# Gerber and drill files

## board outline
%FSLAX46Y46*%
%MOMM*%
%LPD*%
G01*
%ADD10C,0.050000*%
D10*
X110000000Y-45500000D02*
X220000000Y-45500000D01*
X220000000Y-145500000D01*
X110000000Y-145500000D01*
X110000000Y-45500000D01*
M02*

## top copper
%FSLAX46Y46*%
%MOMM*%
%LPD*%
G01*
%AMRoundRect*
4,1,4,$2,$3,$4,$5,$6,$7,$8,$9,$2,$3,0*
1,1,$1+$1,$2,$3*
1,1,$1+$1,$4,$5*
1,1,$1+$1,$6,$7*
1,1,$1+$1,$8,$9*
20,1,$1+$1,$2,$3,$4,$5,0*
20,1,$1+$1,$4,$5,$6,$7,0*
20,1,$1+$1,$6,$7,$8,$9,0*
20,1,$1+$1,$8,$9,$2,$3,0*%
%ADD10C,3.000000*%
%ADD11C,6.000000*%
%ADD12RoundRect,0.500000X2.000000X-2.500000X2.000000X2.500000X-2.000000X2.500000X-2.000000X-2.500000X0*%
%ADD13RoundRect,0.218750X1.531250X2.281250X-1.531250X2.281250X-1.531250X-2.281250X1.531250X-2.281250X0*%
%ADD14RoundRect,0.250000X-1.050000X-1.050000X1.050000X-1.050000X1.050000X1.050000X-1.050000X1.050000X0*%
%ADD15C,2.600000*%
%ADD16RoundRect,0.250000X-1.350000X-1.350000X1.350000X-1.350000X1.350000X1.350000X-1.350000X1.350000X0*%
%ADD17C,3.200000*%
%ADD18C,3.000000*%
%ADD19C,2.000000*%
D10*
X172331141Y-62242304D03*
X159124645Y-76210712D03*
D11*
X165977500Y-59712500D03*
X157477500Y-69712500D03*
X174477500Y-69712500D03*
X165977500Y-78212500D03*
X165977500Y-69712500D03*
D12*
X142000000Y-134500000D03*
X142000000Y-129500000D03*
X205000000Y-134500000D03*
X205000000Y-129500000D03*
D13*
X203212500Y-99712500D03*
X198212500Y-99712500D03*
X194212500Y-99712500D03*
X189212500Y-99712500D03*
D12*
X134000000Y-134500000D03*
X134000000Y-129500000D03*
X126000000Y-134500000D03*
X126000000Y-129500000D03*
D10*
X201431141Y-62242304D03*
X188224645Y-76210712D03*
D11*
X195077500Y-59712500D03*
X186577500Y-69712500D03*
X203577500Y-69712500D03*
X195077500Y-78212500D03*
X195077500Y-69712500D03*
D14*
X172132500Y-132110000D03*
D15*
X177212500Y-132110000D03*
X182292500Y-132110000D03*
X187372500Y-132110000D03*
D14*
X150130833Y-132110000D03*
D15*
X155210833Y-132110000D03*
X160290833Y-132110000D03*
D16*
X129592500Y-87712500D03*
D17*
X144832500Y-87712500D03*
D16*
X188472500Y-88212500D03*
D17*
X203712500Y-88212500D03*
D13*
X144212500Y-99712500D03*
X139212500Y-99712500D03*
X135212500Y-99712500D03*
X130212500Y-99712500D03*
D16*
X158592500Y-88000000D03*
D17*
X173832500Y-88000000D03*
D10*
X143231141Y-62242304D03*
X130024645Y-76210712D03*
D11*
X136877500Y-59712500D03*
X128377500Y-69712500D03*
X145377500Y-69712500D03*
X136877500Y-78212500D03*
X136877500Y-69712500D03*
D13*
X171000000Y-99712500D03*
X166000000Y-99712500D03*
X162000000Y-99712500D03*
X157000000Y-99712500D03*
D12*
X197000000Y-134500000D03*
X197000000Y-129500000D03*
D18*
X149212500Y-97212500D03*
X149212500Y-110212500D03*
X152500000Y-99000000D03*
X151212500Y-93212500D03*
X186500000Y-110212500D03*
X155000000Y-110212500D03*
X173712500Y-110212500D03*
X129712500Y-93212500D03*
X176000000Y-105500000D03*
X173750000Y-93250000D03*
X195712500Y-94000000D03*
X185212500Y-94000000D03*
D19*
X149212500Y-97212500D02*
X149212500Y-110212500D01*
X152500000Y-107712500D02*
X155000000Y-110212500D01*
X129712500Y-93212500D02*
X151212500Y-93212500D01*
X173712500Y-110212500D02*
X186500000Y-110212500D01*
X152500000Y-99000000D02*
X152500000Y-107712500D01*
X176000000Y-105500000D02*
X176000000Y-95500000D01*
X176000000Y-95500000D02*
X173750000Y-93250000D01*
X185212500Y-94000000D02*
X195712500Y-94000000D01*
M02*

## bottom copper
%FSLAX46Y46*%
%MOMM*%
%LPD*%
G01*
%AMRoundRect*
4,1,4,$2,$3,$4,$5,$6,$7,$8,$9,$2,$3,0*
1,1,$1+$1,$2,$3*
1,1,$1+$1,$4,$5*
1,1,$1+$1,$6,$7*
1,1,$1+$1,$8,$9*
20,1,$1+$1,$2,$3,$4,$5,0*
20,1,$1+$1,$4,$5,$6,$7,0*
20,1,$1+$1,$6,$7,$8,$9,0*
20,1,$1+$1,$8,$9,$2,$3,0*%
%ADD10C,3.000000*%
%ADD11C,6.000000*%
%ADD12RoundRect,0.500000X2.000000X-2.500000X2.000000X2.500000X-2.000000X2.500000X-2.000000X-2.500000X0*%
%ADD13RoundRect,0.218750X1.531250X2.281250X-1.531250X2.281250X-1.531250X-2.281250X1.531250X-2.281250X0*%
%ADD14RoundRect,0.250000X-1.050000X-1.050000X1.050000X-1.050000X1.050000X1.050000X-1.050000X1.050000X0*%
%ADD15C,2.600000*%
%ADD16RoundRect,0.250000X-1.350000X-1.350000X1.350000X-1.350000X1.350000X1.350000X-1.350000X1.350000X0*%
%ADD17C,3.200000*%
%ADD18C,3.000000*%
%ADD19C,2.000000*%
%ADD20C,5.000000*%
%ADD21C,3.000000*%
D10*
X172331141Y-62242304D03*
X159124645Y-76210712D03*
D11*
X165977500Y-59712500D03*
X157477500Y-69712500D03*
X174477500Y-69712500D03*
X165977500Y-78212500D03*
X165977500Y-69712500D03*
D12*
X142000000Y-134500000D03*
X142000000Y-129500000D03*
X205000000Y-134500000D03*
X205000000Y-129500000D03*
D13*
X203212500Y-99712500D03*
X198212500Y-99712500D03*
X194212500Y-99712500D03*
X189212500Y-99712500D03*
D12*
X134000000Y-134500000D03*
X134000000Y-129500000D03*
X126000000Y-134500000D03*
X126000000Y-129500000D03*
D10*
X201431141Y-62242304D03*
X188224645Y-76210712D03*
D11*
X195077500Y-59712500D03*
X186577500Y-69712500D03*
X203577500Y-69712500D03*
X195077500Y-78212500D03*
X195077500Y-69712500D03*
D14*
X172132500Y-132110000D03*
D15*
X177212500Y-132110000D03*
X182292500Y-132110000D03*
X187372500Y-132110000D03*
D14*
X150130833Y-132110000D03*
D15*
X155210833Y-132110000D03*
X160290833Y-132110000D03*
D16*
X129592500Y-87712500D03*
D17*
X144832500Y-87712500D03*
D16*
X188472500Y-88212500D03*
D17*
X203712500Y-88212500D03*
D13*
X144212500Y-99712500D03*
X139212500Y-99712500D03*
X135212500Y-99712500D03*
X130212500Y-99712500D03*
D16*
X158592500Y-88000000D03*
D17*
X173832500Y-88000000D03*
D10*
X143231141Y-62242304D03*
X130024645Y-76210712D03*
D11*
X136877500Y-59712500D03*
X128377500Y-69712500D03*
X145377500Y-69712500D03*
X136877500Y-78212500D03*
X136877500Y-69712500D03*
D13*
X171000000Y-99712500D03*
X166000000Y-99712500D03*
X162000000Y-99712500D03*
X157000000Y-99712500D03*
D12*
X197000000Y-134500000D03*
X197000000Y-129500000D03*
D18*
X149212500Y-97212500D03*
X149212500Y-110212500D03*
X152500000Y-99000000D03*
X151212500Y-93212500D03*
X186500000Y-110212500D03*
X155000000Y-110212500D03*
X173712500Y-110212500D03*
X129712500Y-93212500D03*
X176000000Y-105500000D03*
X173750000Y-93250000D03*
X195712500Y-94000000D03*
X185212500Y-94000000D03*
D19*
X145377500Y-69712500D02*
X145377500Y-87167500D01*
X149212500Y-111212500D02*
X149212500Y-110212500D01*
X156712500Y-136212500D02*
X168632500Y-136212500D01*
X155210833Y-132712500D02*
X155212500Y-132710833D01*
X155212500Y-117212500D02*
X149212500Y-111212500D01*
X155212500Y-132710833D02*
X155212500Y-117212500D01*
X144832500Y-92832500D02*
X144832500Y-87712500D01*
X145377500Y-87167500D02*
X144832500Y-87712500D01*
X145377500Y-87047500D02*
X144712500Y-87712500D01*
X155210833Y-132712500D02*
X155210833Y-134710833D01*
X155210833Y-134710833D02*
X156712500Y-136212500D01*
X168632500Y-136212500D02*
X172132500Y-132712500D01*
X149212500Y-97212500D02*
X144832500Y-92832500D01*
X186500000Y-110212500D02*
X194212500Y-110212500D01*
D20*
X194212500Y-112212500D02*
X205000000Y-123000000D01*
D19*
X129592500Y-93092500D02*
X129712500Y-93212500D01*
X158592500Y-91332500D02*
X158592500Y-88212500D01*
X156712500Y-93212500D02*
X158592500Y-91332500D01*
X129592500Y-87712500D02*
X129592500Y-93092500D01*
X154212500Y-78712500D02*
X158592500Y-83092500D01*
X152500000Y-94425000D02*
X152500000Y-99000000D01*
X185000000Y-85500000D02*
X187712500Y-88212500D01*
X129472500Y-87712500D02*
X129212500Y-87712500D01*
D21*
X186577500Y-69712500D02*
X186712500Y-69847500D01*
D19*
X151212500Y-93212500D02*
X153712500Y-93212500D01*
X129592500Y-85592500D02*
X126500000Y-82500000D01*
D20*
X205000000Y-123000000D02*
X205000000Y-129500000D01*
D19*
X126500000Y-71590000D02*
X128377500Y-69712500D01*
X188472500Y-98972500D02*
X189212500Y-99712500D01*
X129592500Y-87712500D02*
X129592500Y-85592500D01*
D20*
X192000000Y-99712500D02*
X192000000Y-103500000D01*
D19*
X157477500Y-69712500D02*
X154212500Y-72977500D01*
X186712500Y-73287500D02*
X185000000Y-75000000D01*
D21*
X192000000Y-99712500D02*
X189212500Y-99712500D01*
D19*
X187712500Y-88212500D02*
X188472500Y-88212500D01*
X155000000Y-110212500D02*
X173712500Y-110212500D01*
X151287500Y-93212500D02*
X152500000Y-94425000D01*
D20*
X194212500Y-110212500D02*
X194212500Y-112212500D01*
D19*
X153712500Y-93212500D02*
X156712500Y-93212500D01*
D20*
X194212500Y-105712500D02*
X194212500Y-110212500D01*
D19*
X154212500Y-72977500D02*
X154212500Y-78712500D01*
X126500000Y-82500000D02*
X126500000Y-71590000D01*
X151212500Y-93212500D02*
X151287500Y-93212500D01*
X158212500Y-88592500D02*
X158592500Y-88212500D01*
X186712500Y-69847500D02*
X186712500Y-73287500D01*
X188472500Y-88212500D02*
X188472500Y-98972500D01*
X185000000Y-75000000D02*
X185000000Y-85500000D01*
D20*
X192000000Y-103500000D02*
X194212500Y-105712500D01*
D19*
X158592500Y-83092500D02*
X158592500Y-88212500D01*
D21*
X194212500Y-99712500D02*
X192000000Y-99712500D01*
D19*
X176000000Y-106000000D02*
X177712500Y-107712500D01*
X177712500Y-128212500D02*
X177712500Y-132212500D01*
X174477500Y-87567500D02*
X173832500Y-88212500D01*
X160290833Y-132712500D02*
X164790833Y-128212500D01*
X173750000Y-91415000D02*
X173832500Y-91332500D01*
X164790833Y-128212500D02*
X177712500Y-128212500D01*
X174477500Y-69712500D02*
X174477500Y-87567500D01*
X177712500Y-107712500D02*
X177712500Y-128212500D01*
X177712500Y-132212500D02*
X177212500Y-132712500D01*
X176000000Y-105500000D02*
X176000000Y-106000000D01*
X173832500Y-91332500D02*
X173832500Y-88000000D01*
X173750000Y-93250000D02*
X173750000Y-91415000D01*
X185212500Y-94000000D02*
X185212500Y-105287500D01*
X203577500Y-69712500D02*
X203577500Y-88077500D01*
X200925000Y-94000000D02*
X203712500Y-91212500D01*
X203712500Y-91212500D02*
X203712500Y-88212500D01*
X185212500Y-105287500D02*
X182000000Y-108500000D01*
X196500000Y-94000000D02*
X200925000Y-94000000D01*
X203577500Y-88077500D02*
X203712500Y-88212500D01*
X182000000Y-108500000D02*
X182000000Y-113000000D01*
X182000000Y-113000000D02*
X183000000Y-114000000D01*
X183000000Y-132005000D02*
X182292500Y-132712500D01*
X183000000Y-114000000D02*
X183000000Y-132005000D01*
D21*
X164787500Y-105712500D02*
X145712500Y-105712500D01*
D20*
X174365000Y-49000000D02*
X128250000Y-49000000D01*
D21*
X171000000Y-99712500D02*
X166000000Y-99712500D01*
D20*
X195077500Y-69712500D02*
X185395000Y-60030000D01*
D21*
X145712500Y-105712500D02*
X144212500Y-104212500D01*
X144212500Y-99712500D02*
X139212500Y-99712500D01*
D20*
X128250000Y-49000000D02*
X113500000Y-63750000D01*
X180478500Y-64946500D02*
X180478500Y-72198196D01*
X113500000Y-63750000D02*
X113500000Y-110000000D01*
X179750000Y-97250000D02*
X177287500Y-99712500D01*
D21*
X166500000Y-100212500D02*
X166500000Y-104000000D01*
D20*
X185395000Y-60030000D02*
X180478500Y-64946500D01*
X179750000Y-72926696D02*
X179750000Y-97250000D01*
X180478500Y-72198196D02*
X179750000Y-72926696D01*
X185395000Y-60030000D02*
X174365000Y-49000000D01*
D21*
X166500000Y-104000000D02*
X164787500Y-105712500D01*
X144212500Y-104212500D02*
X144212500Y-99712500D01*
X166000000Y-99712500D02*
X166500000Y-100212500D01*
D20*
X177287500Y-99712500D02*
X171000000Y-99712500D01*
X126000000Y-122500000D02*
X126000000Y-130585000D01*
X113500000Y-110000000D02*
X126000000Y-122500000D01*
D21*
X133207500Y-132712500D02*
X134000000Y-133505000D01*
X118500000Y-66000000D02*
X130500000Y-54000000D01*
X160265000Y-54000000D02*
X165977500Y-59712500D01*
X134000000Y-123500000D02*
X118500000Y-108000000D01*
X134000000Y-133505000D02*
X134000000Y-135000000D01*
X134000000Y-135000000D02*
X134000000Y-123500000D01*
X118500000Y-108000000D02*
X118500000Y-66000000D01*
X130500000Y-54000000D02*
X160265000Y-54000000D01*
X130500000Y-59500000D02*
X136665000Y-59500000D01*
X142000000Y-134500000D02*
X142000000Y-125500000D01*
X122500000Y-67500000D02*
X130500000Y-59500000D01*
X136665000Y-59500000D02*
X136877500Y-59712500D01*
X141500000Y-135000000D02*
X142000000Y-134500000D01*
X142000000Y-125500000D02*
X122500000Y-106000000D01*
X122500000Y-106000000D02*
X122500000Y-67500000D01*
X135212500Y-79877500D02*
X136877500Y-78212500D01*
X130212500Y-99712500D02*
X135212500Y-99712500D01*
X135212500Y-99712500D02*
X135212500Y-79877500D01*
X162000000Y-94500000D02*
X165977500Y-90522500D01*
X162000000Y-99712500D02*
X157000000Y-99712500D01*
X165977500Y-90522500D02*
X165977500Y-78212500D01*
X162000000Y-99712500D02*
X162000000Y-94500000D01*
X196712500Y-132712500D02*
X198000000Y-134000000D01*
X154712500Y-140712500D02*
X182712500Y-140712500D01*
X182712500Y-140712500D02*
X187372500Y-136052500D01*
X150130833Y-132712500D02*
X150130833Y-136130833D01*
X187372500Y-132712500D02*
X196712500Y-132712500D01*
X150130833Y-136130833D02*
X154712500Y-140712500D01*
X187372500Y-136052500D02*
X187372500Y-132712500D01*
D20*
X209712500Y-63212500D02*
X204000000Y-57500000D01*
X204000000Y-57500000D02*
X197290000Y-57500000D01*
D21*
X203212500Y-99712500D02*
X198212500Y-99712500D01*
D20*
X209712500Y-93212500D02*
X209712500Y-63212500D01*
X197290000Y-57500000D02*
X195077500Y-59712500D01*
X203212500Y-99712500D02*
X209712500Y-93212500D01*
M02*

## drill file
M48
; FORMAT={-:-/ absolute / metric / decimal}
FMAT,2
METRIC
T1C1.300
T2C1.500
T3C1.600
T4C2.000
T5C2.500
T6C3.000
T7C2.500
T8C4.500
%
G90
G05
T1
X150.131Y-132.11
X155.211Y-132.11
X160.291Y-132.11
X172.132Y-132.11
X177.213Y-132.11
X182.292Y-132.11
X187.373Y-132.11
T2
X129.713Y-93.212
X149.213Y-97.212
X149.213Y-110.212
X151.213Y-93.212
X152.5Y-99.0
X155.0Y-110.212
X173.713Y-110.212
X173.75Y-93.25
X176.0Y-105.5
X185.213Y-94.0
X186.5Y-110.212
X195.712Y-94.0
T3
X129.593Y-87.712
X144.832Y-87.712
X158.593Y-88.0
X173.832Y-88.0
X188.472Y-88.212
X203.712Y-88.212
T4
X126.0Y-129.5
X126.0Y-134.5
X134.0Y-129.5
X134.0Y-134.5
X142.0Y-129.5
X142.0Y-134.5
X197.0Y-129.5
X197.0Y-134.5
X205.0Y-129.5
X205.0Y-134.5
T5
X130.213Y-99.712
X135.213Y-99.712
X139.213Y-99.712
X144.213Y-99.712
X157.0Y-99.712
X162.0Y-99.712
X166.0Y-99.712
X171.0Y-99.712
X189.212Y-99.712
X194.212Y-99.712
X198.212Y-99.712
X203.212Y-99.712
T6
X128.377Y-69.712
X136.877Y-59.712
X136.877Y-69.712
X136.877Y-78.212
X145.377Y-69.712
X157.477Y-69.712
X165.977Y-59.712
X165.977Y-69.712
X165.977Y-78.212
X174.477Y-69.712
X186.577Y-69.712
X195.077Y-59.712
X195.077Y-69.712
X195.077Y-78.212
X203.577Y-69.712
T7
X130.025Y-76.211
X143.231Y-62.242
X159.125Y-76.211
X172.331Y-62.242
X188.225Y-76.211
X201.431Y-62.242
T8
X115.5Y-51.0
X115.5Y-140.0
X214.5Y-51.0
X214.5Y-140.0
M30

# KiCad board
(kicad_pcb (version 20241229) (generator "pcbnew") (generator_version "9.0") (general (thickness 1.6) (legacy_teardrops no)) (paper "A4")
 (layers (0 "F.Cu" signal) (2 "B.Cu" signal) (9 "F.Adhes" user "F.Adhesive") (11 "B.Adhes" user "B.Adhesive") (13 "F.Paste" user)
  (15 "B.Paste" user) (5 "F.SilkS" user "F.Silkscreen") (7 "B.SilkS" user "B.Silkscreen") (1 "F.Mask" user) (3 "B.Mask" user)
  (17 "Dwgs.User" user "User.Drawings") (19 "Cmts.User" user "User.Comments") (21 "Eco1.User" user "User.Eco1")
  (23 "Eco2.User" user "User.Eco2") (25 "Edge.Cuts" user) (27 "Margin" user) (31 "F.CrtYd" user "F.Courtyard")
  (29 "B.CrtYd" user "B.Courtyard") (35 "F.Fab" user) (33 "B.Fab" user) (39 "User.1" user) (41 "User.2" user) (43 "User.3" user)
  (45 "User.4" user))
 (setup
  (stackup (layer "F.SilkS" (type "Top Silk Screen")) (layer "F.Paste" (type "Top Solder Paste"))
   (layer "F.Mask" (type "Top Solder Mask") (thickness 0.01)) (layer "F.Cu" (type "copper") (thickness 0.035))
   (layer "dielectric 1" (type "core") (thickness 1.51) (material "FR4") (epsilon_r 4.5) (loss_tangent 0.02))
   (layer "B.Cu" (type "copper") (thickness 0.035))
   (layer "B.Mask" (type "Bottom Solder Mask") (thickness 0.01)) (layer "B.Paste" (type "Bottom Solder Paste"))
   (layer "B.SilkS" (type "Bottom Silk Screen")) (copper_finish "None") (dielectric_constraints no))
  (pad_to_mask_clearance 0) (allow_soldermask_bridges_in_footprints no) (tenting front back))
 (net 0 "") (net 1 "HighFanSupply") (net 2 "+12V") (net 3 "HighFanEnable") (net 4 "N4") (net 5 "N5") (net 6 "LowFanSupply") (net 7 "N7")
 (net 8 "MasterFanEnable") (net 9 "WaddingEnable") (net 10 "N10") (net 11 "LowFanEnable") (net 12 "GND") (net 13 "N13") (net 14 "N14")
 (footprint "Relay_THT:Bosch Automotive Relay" (layer "F.Cu") (at 165.9775 69.4625 180)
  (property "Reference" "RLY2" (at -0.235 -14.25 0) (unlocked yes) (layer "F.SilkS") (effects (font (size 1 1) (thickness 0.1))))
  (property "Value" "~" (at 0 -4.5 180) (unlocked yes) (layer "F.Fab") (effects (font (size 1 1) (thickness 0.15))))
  (pad "" np_thru_hole circle (at -6.353641 7.220196 180) (size 3 3) (drill 2.5) (layers "*.Cu" "*.Mask"))
  (pad "" np_thru_hole circle (at 6.852855 -6.748212 180) (size 3 3) (drill 2.5) (layers "*.Cu" "*.Mask"))
  (pad "30" thru_hole circle (at 0 9.75 180) (size 6 6) (drill 3) (layers "*.Cu" "*.Mask") (remove_unused_layers no) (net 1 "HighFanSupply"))
  (pad "85" thru_hole circle (at 8.5 -0.25 180) (size 6 6) (drill 3) (layers "*.Cu" "*.Mask") (remove_unused_layers no) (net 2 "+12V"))
  (pad "86" thru_hole circle (at -8.5 -0.25 180) (size 6 6) (drill 3) (layers "*.Cu" "*.Mask") (remove_unused_layers no)
   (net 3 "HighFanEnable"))
  (pad "87" thru_hole circle (at 0 -8.75 180) (size 6 6) (drill 3) (layers "*.Cu" "*.Mask") (remove_unused_layers no) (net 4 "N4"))
  (pad "87a" thru_hole circle (at 0 -0.25 180) (size 6 6) (drill 3) (layers "*.Cu" "*.Mask") (remove_unused_layers no) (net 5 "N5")))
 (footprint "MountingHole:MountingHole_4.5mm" (layer "F.Cu") (at 115.5 51)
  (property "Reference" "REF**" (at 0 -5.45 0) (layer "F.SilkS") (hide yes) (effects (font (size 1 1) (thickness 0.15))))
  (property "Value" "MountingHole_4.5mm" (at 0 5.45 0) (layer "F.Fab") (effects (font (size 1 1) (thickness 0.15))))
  (pad "" np_thru_hole circle (at 0 0) (size 4.5 4.5) (drill 4.5) (layers "*.Cu" "*.Mask")))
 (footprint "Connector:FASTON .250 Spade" (layer "F.Cu") (at 142 132 90)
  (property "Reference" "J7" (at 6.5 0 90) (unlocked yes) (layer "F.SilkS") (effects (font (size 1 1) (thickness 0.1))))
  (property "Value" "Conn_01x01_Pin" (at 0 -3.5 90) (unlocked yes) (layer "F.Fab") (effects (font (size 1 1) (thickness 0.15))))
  (pad "1" thru_hole roundrect (at -2.5 0 90) (size 6 5) (drill 2) (layers "*.Cu" "*.Mask") (remove_unused_layers no) (roundrect_rratio 0.1)
   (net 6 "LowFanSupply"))
  (pad "1" thru_hole roundrect (at 2.5 0 90) (size 6 5) (drill 2) (layers "*.Cu" "*.Mask") (remove_unused_layers no) (roundrect_rratio 0.1)
   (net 6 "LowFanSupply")))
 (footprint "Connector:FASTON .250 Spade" (layer "F.Cu") (at 205 132 90)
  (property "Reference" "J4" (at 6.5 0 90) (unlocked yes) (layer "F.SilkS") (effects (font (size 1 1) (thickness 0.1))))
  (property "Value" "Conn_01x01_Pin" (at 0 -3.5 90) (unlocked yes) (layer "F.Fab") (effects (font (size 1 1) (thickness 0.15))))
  (pad "1" thru_hole roundrect (at -2.5 0 90) (size 6 5) (drill 2) (layers "*.Cu" "*.Mask") (remove_unused_layers no) (roundrect_rratio 0.1)
   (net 2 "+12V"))
  (pad "1" thru_hole roundrect (at 2.5 0 90) (size 6 5) (drill 2) (layers "*.Cu" "*.Mask") (remove_unused_layers no) (roundrect_rratio 0.1)
   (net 2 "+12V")))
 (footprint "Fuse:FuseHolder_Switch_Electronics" (layer "F.Cu") (at 196.2125 99.7125 180)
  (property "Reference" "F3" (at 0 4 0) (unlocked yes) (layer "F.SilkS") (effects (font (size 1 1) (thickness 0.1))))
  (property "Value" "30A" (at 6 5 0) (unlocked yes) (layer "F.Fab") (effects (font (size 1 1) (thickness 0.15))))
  (pad "1" thru_hole roundrect (at -7 0 180) (size 3.5 5) (drill 2.5) (layers "*.Cu" "*.Mask") (remove_unused_layers no)
   (roundrect_rratio 0.0625) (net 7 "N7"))
  (pad "1" thru_hole roundrect (at -2 0 180) (size 3.5 5) (drill 2.5) (layers "*.Cu" "*.Mask") (remove_unused_layers no)
   (roundrect_rratio 0.0625) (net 7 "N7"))
  (pad "2" thru_hole roundrect (at 2 0 180) (size 3.5 5) (drill 2.5) (layers "*.Cu" "*.Mask") (remove_unused_layers no)
   (roundrect_rratio 0.0625) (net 2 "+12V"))
  (pad "2" thru_hole roundrect (at 7 0 180) (size 3.5 5) (drill 2.5) (layers "*.Cu" "*.Mask") (remove_unused_layers no)
   (roundrect_rratio 0.0625) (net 2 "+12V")))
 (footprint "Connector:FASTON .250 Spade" (layer "F.Cu") (at 134 132 90)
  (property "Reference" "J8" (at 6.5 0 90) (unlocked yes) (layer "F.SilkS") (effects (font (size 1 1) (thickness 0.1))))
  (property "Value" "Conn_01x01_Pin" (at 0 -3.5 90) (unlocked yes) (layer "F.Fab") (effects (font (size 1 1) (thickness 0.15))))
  (pad "1" thru_hole roundrect (at -2.5 0 90) (size 6 5) (drill 2) (layers "*.Cu" "*.Mask") (remove_unused_layers no) (roundrect_rratio 0.1)
   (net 1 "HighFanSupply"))
  (pad "1" thru_hole roundrect (at 2.5 0 90) (size 6 5) (drill 2) (layers "*.Cu" "*.Mask") (remove_unused_layers no) (roundrect_rratio 0.1)
   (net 1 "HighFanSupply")))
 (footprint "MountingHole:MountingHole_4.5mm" (layer "F.Cu") (at 214.5 140)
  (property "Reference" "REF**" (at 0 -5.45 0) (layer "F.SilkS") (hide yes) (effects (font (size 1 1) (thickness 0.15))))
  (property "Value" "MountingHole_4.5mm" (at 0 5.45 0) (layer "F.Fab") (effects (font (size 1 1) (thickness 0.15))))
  (pad "" np_thru_hole circle (at 0 0) (size 4.5 4.5) (drill 4.5) (layers "*.Cu" "*.Mask")))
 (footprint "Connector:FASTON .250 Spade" (layer "F.Cu") (at 126 132 90)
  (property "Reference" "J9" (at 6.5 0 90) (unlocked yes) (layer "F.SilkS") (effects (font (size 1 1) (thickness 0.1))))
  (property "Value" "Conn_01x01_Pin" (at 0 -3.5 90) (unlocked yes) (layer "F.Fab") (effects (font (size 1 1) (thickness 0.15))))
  (pad "1" thru_hole roundrect (at -2.5 0 90) (size 6 5) (drill 2) (layers "*.Cu" "*.Mask") (remove_unused_layers no) (roundrect_rratio 0.1)
   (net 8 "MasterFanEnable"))
  (pad "1" thru_hole roundrect (at 2.5 0 90) (size 6 5) (drill 2) (layers "*.Cu" "*.Mask") (remove_unused_layers no) (roundrect_rratio 0.1)
   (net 8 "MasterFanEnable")))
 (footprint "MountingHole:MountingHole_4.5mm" (layer "F.Cu") (at 115.5 140)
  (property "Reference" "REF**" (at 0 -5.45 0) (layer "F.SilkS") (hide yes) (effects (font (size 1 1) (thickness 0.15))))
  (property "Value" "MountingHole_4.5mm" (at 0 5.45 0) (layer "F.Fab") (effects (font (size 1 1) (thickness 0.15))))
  (pad "" np_thru_hole circle (at 0 0) (size 4.5 4.5) (drill 4.5) (layers "*.Cu" "*.Mask")))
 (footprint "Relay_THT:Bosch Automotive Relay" (layer "F.Cu") (at 195.0775 69.4625 180)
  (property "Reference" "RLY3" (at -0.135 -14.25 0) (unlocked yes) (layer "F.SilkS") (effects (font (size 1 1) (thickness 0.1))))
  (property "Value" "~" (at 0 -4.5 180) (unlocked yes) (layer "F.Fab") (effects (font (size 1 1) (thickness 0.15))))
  (pad "" np_thru_hole circle (at -6.353641 7.220196 180) (size 3 3) (drill 2.5) (layers "*.Cu" "*.Mask"))
  (pad "" np_thru_hole circle (at 6.852855 -6.748212 180) (size 3 3) (drill 2.5) (layers "*.Cu" "*.Mask"))
  (pad "30" thru_hole circle (at 0 9.75 180) (size 6 6) (drill 3) (layers "*.Cu" "*.Mask") (remove_unused_layers no) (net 7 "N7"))
  (pad "85" thru_hole circle (at 8.5 -0.25 180) (size 6 6) (drill 3) (layers "*.Cu" "*.Mask") (remove_unused_layers no) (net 2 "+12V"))
  (pad "86" thru_hole circle (at -8.5 -0.25 180) (size 6 6) (drill 3) (layers "*.Cu" "*.Mask") (remove_unused_layers no)
   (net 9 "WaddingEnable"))
  (pad "87" thru_hole circle (at 0 -8.75 180) (size 6 6) (drill 3) (layers "*.Cu" "*.Mask") (remove_unused_layers no) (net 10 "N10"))
  (pad "87a" thru_hole circle (at 0 -0.25 180) (size 6 6) (drill 3) (layers "*.Cu" "*.Mask") (remove_unused_layers no)
   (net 8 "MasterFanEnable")))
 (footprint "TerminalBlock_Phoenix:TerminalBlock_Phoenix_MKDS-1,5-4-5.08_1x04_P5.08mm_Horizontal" (layer "F.Cu") (at 172.1325 132.11)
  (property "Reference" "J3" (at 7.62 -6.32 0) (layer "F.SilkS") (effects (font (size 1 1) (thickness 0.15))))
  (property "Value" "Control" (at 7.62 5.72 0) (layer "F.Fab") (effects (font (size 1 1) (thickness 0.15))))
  (pad "1" thru_hole roundrect (at 0 0) (size 2.6 2.6) (drill 1.3) (layers "*.Cu" "*.Mask") (remove_unused_layers no)
   (roundrect_rratio 0.096154) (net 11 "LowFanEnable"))
  (pad "2" thru_hole circle (at 5.08 0) (size 2.6 2.6) (drill 1.3) (layers "*.Cu" "*.Mask") (remove_unused_layers no)
   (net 3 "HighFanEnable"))
  (pad "3" thru_hole circle (at 10.16 0) (size 2.6 2.6) (drill 1.3) (layers "*.Cu" "*.Mask") (remove_unused_layers no)
   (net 9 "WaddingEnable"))
  (pad "4" thru_hole circle (at 15.24 0) (size 2.6 2.6) (drill 1.3) (layers "*.Cu" "*.Mask") (remove_unused_layers no) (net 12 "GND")))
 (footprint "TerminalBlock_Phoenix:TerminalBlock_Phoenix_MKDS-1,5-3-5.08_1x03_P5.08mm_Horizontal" (layer "F.Cu") (at 150.130833 132.11)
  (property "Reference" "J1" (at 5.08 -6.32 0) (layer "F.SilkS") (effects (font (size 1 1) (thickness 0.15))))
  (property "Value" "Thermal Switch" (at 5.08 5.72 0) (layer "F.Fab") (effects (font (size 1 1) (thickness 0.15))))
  (pad "1" thru_hole roundrect (at 0 0) (size 2.6 2.6) (drill 1.3) (layers "*.Cu" "*.Mask") (remove_unused_layers no)
   (roundrect_rratio 0.096154) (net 12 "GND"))
  (pad "2" thru_hole circle (at 5.08 0) (size 2.6 2.6) (drill 1.3) (layers "*.Cu" "*.Mask") (remove_unused_layers no)
   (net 11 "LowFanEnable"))
  (pad "3" thru_hole circle (at 10.16 0) (size 2.6 2.6) (drill 1.3) (layers "*.Cu" "*.Mask") (remove_unused_layers no)
   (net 3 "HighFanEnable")))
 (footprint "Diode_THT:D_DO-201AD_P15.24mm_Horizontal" (layer "F.Cu") (at 129.5925 87.7125)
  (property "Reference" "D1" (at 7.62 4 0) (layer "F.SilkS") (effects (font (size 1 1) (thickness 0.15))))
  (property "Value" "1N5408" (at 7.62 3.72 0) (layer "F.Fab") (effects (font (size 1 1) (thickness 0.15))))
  (pad "1" thru_hole roundrect (at 0 0) (size 3.2 3.2) (drill 1.6) (layers "*.Cu" "*.Mask") (remove_unused_layers no)
   (roundrect_rratio 0.078125) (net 2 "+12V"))
  (pad "2" thru_hole circle (at 15.24 0) (size 3.2 3.2) (drill 1.6) (layers "*.Cu" "*.Mask") (remove_unused_layers no)
   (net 11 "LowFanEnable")))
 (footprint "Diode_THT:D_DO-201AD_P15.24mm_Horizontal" (layer "F.Cu") (at 188.4725 88.2125)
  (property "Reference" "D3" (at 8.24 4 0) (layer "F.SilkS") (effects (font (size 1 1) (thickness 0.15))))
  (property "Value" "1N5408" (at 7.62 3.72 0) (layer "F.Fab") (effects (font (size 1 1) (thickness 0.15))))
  (pad "1" thru_hole roundrect (at 0 0) (size 3.2 3.2) (drill 1.6) (layers "*.Cu" "*.Mask") (remove_unused_layers no)
   (roundrect_rratio 0.078125) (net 2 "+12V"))
  (pad "2" thru_hole circle (at 15.24 0) (size 3.2 3.2) (drill 1.6) (layers "*.Cu" "*.Mask") (remove_unused_layers no)
   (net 9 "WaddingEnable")))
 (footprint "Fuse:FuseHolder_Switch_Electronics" (layer "F.Cu") (at 137.2125 99.7125 180)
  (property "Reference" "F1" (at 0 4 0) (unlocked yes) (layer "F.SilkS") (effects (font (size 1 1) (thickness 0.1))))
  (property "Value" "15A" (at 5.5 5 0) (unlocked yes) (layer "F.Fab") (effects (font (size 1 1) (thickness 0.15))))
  (pad "1" thru_hole roundrect (at -7 0 180) (size 3.5 5) (drill 2.5) (layers "*.Cu" "*.Mask") (remove_unused_layers no)
   (roundrect_rratio 0.0625) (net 8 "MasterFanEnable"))
  (pad "1" thru_hole roundrect (at -2 0 180) (size 3.5 5) (drill 2.5) (layers "*.Cu" "*.Mask") (remove_unused_layers no)
   (roundrect_rratio 0.0625) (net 8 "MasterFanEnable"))
  (pad "2" thru_hole roundrect (at 2 0 180) (size 3.5 5) (drill 2.5) (layers "*.Cu" "*.Mask") (remove_unused_layers no)
   (roundrect_rratio 0.0625) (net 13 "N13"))
  (pad "2" thru_hole roundrect (at 7 0 180) (size 3.5 5) (drill 2.5) (layers "*.Cu" "*.Mask") (remove_unused_layers no)
   (roundrect_rratio 0.0625) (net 13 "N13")))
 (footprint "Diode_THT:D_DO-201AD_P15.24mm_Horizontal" (layer "F.Cu") (at 158.5925 88)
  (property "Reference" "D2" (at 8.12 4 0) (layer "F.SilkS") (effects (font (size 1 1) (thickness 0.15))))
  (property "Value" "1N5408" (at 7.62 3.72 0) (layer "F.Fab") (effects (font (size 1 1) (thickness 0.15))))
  (pad "1" thru_hole roundrect (at 0 0) (size 3.2 3.2) (drill 1.6) (layers "*.Cu" "*.Mask") (remove_unused_layers no)
   (roundrect_rratio 0.078125) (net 2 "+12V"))
  (pad "2" thru_hole circle (at 15.24 0) (size 3.2 3.2) (drill 1.6) (layers "*.Cu" "*.Mask") (remove_unused_layers no)
   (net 3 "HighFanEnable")))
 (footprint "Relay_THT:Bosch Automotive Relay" (layer "F.Cu") (at 136.8775 69.4625 180)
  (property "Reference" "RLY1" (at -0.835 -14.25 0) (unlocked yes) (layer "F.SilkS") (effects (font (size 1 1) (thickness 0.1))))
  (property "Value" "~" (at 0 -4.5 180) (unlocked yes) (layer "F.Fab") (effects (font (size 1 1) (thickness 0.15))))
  (pad "" np_thru_hole circle (at -6.353641 7.220196 180) (size 3 3) (drill 2.5) (layers "*.Cu" "*.Mask"))
  (pad "" np_thru_hole circle (at 6.852855 -6.748212 180) (size 3 3) (drill 2.5) (layers "*.Cu" "*.Mask"))
  (pad "30" thru_hole circle (at 0 9.75 180) (size 6 6) (drill 3) (layers "*.Cu" "*.Mask") (remove_unused_layers no) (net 6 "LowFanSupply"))
  (pad "85" thru_hole circle (at 8.5 -0.25 180) (size 6 6) (drill 3) (layers "*.Cu" "*.Mask") (remove_unused_layers no) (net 2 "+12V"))
  (pad "86" thru_hole circle (at -8.5 -0.25 180) (size 6 6) (drill 3) (layers "*.Cu" "*.Mask") (remove_unused_layers no)
   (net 11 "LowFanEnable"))
  (pad "87" thru_hole circle (at 0 -8.75 180) (size 6 6) (drill 3) (layers "*.Cu" "*.Mask") (remove_unused_layers no) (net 13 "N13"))
  (pad "87a" thru_hole circle (at 0 -0.25 180) (size 6 6) (drill 3) (layers "*.Cu" "*.Mask") (remove_unused_layers no) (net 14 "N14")))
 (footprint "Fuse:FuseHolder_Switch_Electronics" (layer "F.Cu") (at 164 99.7125 180)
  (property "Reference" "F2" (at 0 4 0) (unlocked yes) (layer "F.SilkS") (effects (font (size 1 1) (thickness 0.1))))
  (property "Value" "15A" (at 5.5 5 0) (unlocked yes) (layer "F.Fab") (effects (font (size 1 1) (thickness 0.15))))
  (pad "1" thru_hole roundrect (at -7 0 180) (size 3.5 5) (drill 2.5) (layers "*.Cu" "*.Mask") (remove_unused_layers no)
   (roundrect_rratio 0.0625) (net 8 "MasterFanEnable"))
  (pad "1" thru_hole roundrect (at -2 0 180) (size 3.5 5) (drill 2.5) (layers "*.Cu" "*.Mask") (remove_unused_layers no)
   (roundrect_rratio 0.0625) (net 8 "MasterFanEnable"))
  (pad "2" thru_hole roundrect (at 2 0 180) (size 3.5 5) (drill 2.5) (layers "*.Cu" "*.Mask") (remove_unused_layers no)
   (roundrect_rratio 0.0625) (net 4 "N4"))
  (pad "2" thru_hole roundrect (at 7 0 180) (size 3.5 5) (drill 2.5) (layers "*.Cu" "*.Mask") (remove_unused_layers no)
   (roundrect_rratio 0.0625) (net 4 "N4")))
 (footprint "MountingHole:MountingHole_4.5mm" (layer "F.Cu") (at 214.5 51)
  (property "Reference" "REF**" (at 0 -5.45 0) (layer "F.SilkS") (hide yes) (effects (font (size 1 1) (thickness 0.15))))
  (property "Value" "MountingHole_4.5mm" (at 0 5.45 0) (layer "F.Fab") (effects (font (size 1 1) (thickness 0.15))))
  (pad "" np_thru_hole circle (at 0 0) (size 4.5 4.5) (drill 4.5) (layers "*.Cu" "*.Mask")))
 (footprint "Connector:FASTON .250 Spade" (layer "F.Cu") (at 197 132 90)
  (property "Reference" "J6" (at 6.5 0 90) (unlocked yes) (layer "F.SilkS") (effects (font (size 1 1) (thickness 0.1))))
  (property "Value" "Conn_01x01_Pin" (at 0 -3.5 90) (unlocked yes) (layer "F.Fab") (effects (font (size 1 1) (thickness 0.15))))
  (pad "1" thru_hole roundrect (at -2.5 0 90) (size 6 5) (drill 2) (layers "*.Cu" "*.Mask") (remove_unused_layers no) (roundrect_rratio 0.1)
   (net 12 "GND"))
  (pad "1" thru_hole roundrect (at 2.5 0 90) (size 6 5) (drill 2) (layers "*.Cu" "*.Mask") (remove_unused_layers no) (roundrect_rratio 0.1)
   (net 12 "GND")))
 (gr_rect (start 110 45.5) (end 220 145.5) (stroke (width 0.05) (type solid)) (fill no) (layer "Edge.Cuts"))
 (segment (start 149.2125 97.2125) (end 149.2125 110.2125) (width 2) (layer "F.Cu") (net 11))
 (via (at 149.2125 97.2125) (size 3) (drill 1.5) (layers "F.Cu" "B.Cu")
  (teardrops (best_length_ratio 0.5) (max_length 1) (best_width_ratio 1) (max_width 2) (curved_edges no) (filter_ratio 0.9) (enabled yes)
   (allow_two_segments yes) (prefer_zone_connections yes))
  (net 11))
 (via (at 149.2125 110.2125) (size 3) (drill 1.5) (layers "F.Cu" "B.Cu")
  (teardrops (best_length_ratio 0.5) (max_length 1) (best_width_ratio 1) (max_width 2) (curved_edges no) (filter_ratio 0.9) (enabled yes)
   (allow_two_segments yes) (prefer_zone_connections yes))
  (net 11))
 (segment (start 145.3775 69.7125) (end 145.3775 87.1675) (width 2) (layer "B.Cu") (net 11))
 (segment (start 149.2125 111.2125) (end 149.2125 110.2125) (width 2) (layer "B.Cu") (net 11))
 (segment (start 156.7125 136.2125) (end 168.6325 136.2125) (width 2) (layer "B.Cu") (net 11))
 (segment (start 155.210833 132.7125) (end 155.2125 132.710833) (width 2) (layer "B.Cu") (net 11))
 (segment (start 155.2125 117.2125) (end 149.2125 111.2125) (width 2) (layer "B.Cu") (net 11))
 (segment (start 155.2125 132.710833) (end 155.2125 117.2125) (width 2) (layer "B.Cu") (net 11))
 (segment (start 144.8325 92.8325) (end 144.8325 87.7125) (width 2) (layer "B.Cu") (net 11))
 (segment (start 145.3775 87.1675) (end 144.8325 87.7125) (width 2) (layer "B.Cu") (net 11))
 (segment (start 145.3775 87.0475) (end 144.7125 87.7125) (width 2) (layer "B.Cu") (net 11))
 (segment (start 155.210833 132.7125) (end 155.210833 134.710833) (width 2) (layer "B.Cu") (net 11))
 (segment (start 155.210833 134.710833) (end 156.7125 136.2125) (width 2) (layer "B.Cu") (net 11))
 (segment (start 168.6325 136.2125) (end 172.1325 132.7125) (width 2) (layer "B.Cu") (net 11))
 (segment (start 149.2125 97.2125) (end 144.8325 92.8325) (width 2) (layer "B.Cu") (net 11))
 (segment (start 152.5 107.7125) (end 155 110.2125) (width 2) (layer "F.Cu") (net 2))
 (segment (start 129.7125 93.2125) (end 151.2125 93.2125) (width 2) (layer "F.Cu") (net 2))
 (segment (start 173.7125 110.2125) (end 186.5 110.2125) (width 2) (layer "F.Cu") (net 2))
 (segment (start 152.5 99) (end 152.5 107.7125) (width 2) (layer "F.Cu") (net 2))
 (via (at 152.5 99) (size 3) (drill 1.5) (layers "F.Cu" "B.Cu")
  (teardrops (best_length_ratio 0.5) (max_length 1) (best_width_ratio 1) (max_width 2) (curved_edges no) (filter_ratio 0.9) (enabled yes)
   (allow_two_segments yes) (prefer_zone_connections yes))
  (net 2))
 (via (at 151.2125 93.2125) (size 3) (drill 1.5) (layers "F.Cu" "B.Cu")
  (teardrops (best_length_ratio 0.5) (max_length 1) (best_width_ratio 1) (max_width 2) (curved_edges no) (filter_ratio 0.9) (enabled yes)
   (allow_two_segments yes) (prefer_zone_connections yes))
  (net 2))
 (via (at 186.5 110.2125) (size 3) (drill 1.5) (layers "F.Cu" "B.Cu")
  (teardrops (best_length_ratio 0.5) (max_length 1) (best_width_ratio 1) (max_width 2) (curved_edges no) (filter_ratio 0.9) (enabled yes)
   (allow_two_segments yes) (prefer_zone_connections yes))
  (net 2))
 (via (at 155 110.2125) (size 3) (drill 1.5) (layers "F.Cu" "B.Cu")
  (teardrops (best_length_ratio 0.5) (max_length 1) (best_width_ratio 1) (max_width 2) (curved_edges no) (filter_ratio 0.9) (enabled yes)
   (allow_two_segments yes) (prefer_zone_connections yes))
  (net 2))
 (via (at 173.7125 110.2125) (size 3) (drill 1.5) (layers "F.Cu" "B.Cu")
  (teardrops (best_length_ratio 0.5) (max_length 1) (best_width_ratio 1) (max_width 2) (curved_edges no) (filter_ratio 0.9) (enabled yes)
   (allow_two_segments yes) (prefer_zone_connections yes))
  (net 2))
 (via (at 129.7125 93.2125) (size 3) (drill 1.5) (layers "F.Cu" "B.Cu")
  (teardrops (best_length_ratio 0.5) (max_length 1) (best_width_ratio 1) (max_width 2) (curved_edges no) (filter_ratio 0.9) (enabled yes)
   (allow_two_segments yes) (prefer_zone_connections yes))
  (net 2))
 (segment (start 186.5 110.2125) (end 194.2125 110.2125) (width 2) (layer "B.Cu") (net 2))
 (segment (start 194.2125 112.2125) (end 205 123) (width 5) (layer "B.Cu") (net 2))
 (segment (start 129.5925 93.0925) (end 129.7125 93.2125) (width 2) (layer "B.Cu") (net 2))
 (segment (start 158.5925 91.3325) (end 158.5925 88.2125) (width 2) (layer "B.Cu") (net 2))
 (segment (start 156.7125 93.2125) (end 158.5925 91.3325) (width 2) (layer "B.Cu") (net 2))
 (segment (start 129.5925 87.7125) (end 129.5925 93.0925) (width 2) (layer "B.Cu") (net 2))
 (segment (start 154.2125 78.7125) (end 158.5925 83.0925) (width 2) (layer "B.Cu") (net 2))
 (segment (start 152.5 94.425) (end 152.5 99) (width 2) (layer "B.Cu") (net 2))
 (segment (start 185 85.5) (end 187.7125 88.2125) (width 2) (layer "B.Cu") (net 2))
 (segment (start 129.4725 87.7125) (end 129.2125 87.7125) (width 2) (layer "B.Cu") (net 2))
 (segment (start 186.5775 69.7125) (end 186.7125 69.8475) (width 3) (layer "B.Cu") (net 2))
 (segment (start 151.2125 93.2125) (end 153.7125 93.2125) (width 2) (layer "B.Cu") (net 2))
 (segment (start 129.5925 85.5925) (end 126.5 82.5) (width 2) (layer "B.Cu") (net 2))
 (segment (start 205 123) (end 205 129.5) (width 5) (layer "B.Cu") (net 2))
 (segment (start 126.5 71.59) (end 128.3775 69.7125) (width 2) (layer "B.Cu") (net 2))
 (segment (start 188.4725 98.9725) (end 189.2125 99.7125) (width 2) (layer "B.Cu") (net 2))
 (segment (start 129.5925 87.7125) (end 129.5925 85.5925) (width 2) (layer "B.Cu") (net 2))
 (segment (start 192 99.7125) (end 192 103.5) (width 5) (layer "B.Cu") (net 2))
 (segment (start 157.4775 69.7125) (end 154.2125 72.9775) (width 2) (layer "B.Cu") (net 2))
 (segment (start 186.7125 73.2875) (end 185 75) (width 2) (layer "B.Cu") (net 2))
 (segment (start 192 99.7125) (end 189.2125 99.7125) (width 3) (layer "B.Cu") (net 2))
 (segment (start 187.7125 88.2125) (end 188.4725 88.2125) (width 2) (layer "B.Cu") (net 2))
 (segment (start 155 110.2125) (end 173.7125 110.2125) (width 2) (layer "B.Cu") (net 2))
 (segment (start 151.2875 93.2125) (end 152.5 94.425) (width 2) (layer "B.Cu") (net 2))
 (segment (start 194.2125 110.2125) (end 194.2125 112.2125) (width 5) (layer "B.Cu") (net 2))
 (segment (start 153.7125 93.2125) (end 156.7125 93.2125) (width 2) (layer "B.Cu") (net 2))
 (segment (start 194.2125 105.7125) (end 194.2125 110.2125) (width 5) (layer "B.Cu") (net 2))
 (segment (start 154.2125 72.9775) (end 154.2125 78.7125) (width 2) (layer "B.Cu") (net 2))
 (segment (start 126.5 82.5) (end 126.5 71.59) (width 2) (layer "B.Cu") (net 2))
 (segment (start 151.2125 93.2125) (end 151.2875 93.2125) (width 2) (layer "B.Cu") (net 2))
 (segment (start 158.2125 88.5925) (end 158.5925 88.2125) (width 2) (layer "B.Cu") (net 2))
 (segment (start 186.7125 69.8475) (end 186.7125 73.2875) (width 2) (layer "B.Cu") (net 2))
 (segment (start 188.4725 88.2125) (end 188.4725 98.9725) (width 2) (layer "B.Cu") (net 2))
 (segment (start 185 75) (end 185 85.5) (width 2) (layer "B.Cu") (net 2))
 (segment (start 192 103.5) (end 194.2125 105.7125) (width 5) (layer "B.Cu") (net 2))
 (segment (start 158.5925 83.0925) (end 158.5925 88.2125) (width 2) (layer "B.Cu") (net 2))
 (segment (start 194.2125 99.7125) (end 192 99.7125) (width 3) (layer "B.Cu") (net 2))
 (segment (start 176 105.5) (end 176 95.5) (width 2) (layer "F.Cu") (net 3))
 (segment (start 176 95.5) (end 173.75 93.25) (width 2) (layer "F.Cu") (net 3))
 (via (at 176 105.5) (size 3) (drill 1.5) (layers "F.Cu" "B.Cu")
  (teardrops (best_length_ratio 0.5) (max_length 1) (best_width_ratio 1) (max_width 2) (curved_edges no) (filter_ratio 0.9) (enabled yes)
   (allow_two_segments yes) (prefer_zone_connections yes))
  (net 3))
 (via (at 173.75 93.25) (size 3) (drill 1.5) (layers "F.Cu" "B.Cu")
  (teardrops (best_length_ratio 0.5) (max_length 1) (best_width_ratio 1) (max_width 2) (curved_edges no) (filter_ratio 0.9) (enabled yes)
   (allow_two_segments yes) (prefer_zone_connections yes))
  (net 3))
 (segment (start 176 106) (end 177.7125 107.7125) (width 2) (layer "B.Cu") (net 3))
 (segment (start 177.7125 128.2125) (end 177.7125 132.2125) (width 2) (layer "B.Cu") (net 3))
 (segment (start 174.4775 87.5675) (end 173.8325 88.2125) (width 2) (layer "B.Cu") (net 3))
 (segment (start 160.290833 132.7125) (end 164.790833 128.2125) (width 2) (layer "B.Cu") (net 3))
 (segment (start 173.75 91.415) (end 173.8325 91.3325) (width 2) (layer "B.Cu") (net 3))
 (segment (start 164.790833 128.2125) (end 177.7125 128.2125) (width 2) (layer "B.Cu") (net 3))
 (segment (start 174.4775 69.7125) (end 174.4775 87.5675) (width 2) (layer "B.Cu") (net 3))
 (segment (start 177.7125 107.7125) (end 177.7125 128.2125) (width 2) (layer "B.Cu") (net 3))
 (segment (start 177.7125 132.2125) (end 177.2125 132.7125) (width 2) (layer "B.Cu") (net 3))
 (segment (start 176 105.5) (end 176 106) (width 2) (layer "B.Cu") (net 3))
 (segment (start 173.8325 91.3325) (end 173.8325 88) (width 2) (layer "B.Cu") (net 3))
 (segment (start 173.75 93.25) (end 173.75 91.415) (width 2) (layer "B.Cu") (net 3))
 (segment (start 185.2125 94) (end 195.7125 94) (width 2) (layer "F.Cu") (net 9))
 (via (at 195.7125 94) (size 3) (drill 1.5) (layers "F.Cu" "B.Cu")
  (teardrops (best_length_ratio 0.5) (max_length 1) (best_width_ratio 1) (max_width 2) (curved_edges no) (filter_ratio 0.9) (enabled yes)
   (allow_two_segments yes) (prefer_zone_connections yes))
  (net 9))
 (via (at 185.2125 94) (size 3) (drill 1.5) (layers "F.Cu" "B.Cu")
  (teardrops (best_length_ratio 0.5) (max_length 1) (best_width_ratio 1) (max_width 2) (curved_edges no) (filter_ratio 0.9) (enabled yes)
   (allow_two_segments yes) (prefer_zone_connections yes))
  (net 9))
 (segment (start 185.2125 94) (end 185.2125 105.2875) (width 2) (layer "B.Cu") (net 9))
 (segment (start 203.5775 69.7125) (end 203.5775 88.0775) (width 2) (layer "B.Cu") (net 9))
 (segment (start 200.925 94) (end 203.7125 91.2125) (width 2) (layer "B.Cu") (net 9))
 (segment (start 203.7125 91.2125) (end 203.7125 88.2125) (width 2) (layer "B.Cu") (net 9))
 (segment (start 185.2125 105.2875) (end 182 108.5) (width 2) (layer "B.Cu") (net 9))
 (segment (start 196.5 94) (end 200.925 94) (width 2) (layer "B.Cu") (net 9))
 (segment (start 203.5775 88.0775) (end 203.7125 88.2125) (width 2) (layer "B.Cu") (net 9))
 (segment (start 182 108.5) (end 182 113) (width 2) (layer "B.Cu") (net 9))
 (segment (start 182 113) (end 183 114) (width 2) (layer "B.Cu") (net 9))
 (segment (start 183 132.005) (end 182.2925 132.7125) (width 2) (layer "B.Cu") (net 9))
 (segment (start 183 114) (end 183 132.005) (width 2) (layer "B.Cu") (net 9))
 (segment (start 164.7875 105.7125) (end 145.7125 105.7125) (width 3) (layer "B.Cu") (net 8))
 (segment (start 174.365 49) (end 128.25 49) (width 5) (layer "B.Cu") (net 8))
 (segment (start 171 99.7125) (end 166 99.7125) (width 3) (layer "B.Cu") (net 8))
 (segment (start 195.0775 69.7125) (end 185.395 60.03) (width 5) (layer "B.Cu") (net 8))
 (segment (start 145.7125 105.7125) (end 144.2125 104.2125) (width 3) (layer "B.Cu") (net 8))
 (segment (start 144.2125 99.7125) (end 139.2125 99.7125) (width 3) (layer "B.Cu") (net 8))
 (segment (start 128.25 49) (end 113.5 63.75) (width 5) (layer "B.Cu") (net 8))
 (segment (start 180.4785 64.9465) (end 180.4785 72.198196) (width 5) (layer "B.Cu") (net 8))
 (segment (start 113.5 63.75) (end 113.5 110) (width 5) (layer "B.Cu") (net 8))
 (segment (start 179.75 97.25) (end 177.2875 99.7125) (width 5) (layer "B.Cu") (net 8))
 (segment (start 166.5 100.2125) (end 166.5 104) (width 3) (layer "B.Cu") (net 8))
 (segment (start 185.395 60.03) (end 180.4785 64.9465) (width 5) (layer "B.Cu") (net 8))
 (segment (start 179.75 72.926696) (end 179.75 97.25) (width 5) (layer "B.Cu") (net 8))
 (segment (start 180.4785 72.198196) (end 179.75 72.926696) (width 5) (layer "B.Cu") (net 8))
 (segment (start 185.395 60.03) (end 174.365 49) (width 5) (layer "B.Cu") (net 8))
 (segment (start 166.5 104) (end 164.7875 105.7125) (width 3) (layer "B.Cu") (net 8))
 (segment (start 144.2125 104.2125) (end 144.2125 99.7125) (width 3) (layer "B.Cu") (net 8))
 (segment (start 166 99.7125) (end 166.5 100.2125) (width 3) (layer "B.Cu") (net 8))
 (segment (start 177.2875 99.7125) (end 171 99.7125) (width 5) (layer "B.Cu") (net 8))
 (segment (start 126 122.5) (end 126 130.585) (width 5) (layer "B.Cu") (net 8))
 (segment (start 113.5 110) (end 126 122.5) (width 5) (layer "B.Cu") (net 8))
 (segment (start 133.2075 132.7125) (end 134 133.505) (width 3) (layer "B.Cu") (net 1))
 (segment (start 118.5 66) (end 130.5 54) (width 3) (layer "B.Cu") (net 1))
 (segment (start 160.265 54) (end 165.9775 59.7125) (width 3) (layer "B.Cu") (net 1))
 (segment (start 134 123.5) (end 118.5 108) (width 3) (layer "B.Cu") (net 1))
 (segment (start 134 133.505) (end 134 135) (width 3) (layer "B.Cu") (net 1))
 (segment (start 134 135) (end 134 123.5) (width 3) (layer "B.Cu") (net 1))
 (segment (start 118.5 108) (end 118.5 66) (width 3) (layer "B.Cu") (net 1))
 (segment (start 130.5 54) (end 160.265 54) (width 3) (layer "B.Cu") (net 1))
 (segment (start 130.5 59.5) (end 136.665 59.5) (width 3) (layer "B.Cu") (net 6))
 (segment (start 142 134.5) (end 142 125.5) (width 3) (layer "B.Cu") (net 6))
 (segment (start 122.5 67.5) (end 130.5 59.5) (width 3) (layer "B.Cu") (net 6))
 (segment (start 136.665 59.5) (end 136.8775 59.7125) (width 3) (layer "B.Cu") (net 6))
 (segment (start 141.5 135) (end 142 134.5) (width 3) (layer "B.Cu") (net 6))
 (segment (start 142 125.5) (end 122.5 106) (width 3) (layer "B.Cu") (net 6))
 (segment (start 122.5 106) (end 122.5 67.5) (width 3) (layer "B.Cu") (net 6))
 (segment (start 135.2125 79.8775) (end 136.8775 78.2125) (width 3) (layer "B.Cu") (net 13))
 (segment (start 130.2125 99.7125) (end 135.2125 99.7125) (width 3) (layer "B.Cu") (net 13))
 (segment (start 135.2125 99.7125) (end 135.2125 79.8775) (width 3) (layer "B.Cu") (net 13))
 (segment (start 162 94.5) (end 165.9775 90.5225) (width 3) (layer "B.Cu") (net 4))
 (segment (start 162 99.7125) (end 157 99.7125) (width 3) (layer "B.Cu") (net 4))
 (segment (start 165.9775 90.5225) (end 165.9775 78.2125) (width 3) (layer "B.Cu") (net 4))
 (segment (start 162 99.7125) (end 162 94.5) (width 3) (layer "B.Cu") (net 4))
 (segment (start 196.7125 132.7125) (end 198 134) (width 3) (layer "B.Cu") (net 12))
 (segment (start 154.7125 140.7125) (end 182.7125 140.7125) (width 3) (layer "B.Cu") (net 12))
 (segment (start 182.7125 140.7125) (end 187.3725 136.0525) (width 3) (layer "B.Cu") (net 12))
 (segment (start 150.130833 132.7125) (end 150.130833 136.130833) (width 3) (layer "B.Cu") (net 12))
 (segment (start 187.3725 132.7125) (end 196.7125 132.7125) (width 3) (layer "B.Cu") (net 12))
 (segment (start 150.130833 136.130833) (end 154.7125 140.7125) (width 3) (layer "B.Cu") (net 12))
 (segment (start 187.3725 136.0525) (end 187.3725 132.7125) (width 3) (layer "B.Cu") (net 12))
 (segment (start 209.7125 63.2125) (end 204 57.5) (width 5) (layer "B.Cu") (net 7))
 (segment (start 204 57.5) (end 197.29 57.5) (width 5) (layer "B.Cu") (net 7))
 (segment (start 203.2125 99.7125) (end 198.2125 99.7125) (width 3) (layer "B.Cu") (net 7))
 (segment (start 209.7125 93.2125) (end 209.7125 63.2125) (width 5) (layer "B.Cu") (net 7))
 (segment (start 197.29 57.5) (end 195.0775 59.7125) (width 5) (layer "B.Cu") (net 7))
 (segment (start 203.2125 99.7125) (end 209.7125 93.2125) (width 5) (layer "B.Cu") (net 7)))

